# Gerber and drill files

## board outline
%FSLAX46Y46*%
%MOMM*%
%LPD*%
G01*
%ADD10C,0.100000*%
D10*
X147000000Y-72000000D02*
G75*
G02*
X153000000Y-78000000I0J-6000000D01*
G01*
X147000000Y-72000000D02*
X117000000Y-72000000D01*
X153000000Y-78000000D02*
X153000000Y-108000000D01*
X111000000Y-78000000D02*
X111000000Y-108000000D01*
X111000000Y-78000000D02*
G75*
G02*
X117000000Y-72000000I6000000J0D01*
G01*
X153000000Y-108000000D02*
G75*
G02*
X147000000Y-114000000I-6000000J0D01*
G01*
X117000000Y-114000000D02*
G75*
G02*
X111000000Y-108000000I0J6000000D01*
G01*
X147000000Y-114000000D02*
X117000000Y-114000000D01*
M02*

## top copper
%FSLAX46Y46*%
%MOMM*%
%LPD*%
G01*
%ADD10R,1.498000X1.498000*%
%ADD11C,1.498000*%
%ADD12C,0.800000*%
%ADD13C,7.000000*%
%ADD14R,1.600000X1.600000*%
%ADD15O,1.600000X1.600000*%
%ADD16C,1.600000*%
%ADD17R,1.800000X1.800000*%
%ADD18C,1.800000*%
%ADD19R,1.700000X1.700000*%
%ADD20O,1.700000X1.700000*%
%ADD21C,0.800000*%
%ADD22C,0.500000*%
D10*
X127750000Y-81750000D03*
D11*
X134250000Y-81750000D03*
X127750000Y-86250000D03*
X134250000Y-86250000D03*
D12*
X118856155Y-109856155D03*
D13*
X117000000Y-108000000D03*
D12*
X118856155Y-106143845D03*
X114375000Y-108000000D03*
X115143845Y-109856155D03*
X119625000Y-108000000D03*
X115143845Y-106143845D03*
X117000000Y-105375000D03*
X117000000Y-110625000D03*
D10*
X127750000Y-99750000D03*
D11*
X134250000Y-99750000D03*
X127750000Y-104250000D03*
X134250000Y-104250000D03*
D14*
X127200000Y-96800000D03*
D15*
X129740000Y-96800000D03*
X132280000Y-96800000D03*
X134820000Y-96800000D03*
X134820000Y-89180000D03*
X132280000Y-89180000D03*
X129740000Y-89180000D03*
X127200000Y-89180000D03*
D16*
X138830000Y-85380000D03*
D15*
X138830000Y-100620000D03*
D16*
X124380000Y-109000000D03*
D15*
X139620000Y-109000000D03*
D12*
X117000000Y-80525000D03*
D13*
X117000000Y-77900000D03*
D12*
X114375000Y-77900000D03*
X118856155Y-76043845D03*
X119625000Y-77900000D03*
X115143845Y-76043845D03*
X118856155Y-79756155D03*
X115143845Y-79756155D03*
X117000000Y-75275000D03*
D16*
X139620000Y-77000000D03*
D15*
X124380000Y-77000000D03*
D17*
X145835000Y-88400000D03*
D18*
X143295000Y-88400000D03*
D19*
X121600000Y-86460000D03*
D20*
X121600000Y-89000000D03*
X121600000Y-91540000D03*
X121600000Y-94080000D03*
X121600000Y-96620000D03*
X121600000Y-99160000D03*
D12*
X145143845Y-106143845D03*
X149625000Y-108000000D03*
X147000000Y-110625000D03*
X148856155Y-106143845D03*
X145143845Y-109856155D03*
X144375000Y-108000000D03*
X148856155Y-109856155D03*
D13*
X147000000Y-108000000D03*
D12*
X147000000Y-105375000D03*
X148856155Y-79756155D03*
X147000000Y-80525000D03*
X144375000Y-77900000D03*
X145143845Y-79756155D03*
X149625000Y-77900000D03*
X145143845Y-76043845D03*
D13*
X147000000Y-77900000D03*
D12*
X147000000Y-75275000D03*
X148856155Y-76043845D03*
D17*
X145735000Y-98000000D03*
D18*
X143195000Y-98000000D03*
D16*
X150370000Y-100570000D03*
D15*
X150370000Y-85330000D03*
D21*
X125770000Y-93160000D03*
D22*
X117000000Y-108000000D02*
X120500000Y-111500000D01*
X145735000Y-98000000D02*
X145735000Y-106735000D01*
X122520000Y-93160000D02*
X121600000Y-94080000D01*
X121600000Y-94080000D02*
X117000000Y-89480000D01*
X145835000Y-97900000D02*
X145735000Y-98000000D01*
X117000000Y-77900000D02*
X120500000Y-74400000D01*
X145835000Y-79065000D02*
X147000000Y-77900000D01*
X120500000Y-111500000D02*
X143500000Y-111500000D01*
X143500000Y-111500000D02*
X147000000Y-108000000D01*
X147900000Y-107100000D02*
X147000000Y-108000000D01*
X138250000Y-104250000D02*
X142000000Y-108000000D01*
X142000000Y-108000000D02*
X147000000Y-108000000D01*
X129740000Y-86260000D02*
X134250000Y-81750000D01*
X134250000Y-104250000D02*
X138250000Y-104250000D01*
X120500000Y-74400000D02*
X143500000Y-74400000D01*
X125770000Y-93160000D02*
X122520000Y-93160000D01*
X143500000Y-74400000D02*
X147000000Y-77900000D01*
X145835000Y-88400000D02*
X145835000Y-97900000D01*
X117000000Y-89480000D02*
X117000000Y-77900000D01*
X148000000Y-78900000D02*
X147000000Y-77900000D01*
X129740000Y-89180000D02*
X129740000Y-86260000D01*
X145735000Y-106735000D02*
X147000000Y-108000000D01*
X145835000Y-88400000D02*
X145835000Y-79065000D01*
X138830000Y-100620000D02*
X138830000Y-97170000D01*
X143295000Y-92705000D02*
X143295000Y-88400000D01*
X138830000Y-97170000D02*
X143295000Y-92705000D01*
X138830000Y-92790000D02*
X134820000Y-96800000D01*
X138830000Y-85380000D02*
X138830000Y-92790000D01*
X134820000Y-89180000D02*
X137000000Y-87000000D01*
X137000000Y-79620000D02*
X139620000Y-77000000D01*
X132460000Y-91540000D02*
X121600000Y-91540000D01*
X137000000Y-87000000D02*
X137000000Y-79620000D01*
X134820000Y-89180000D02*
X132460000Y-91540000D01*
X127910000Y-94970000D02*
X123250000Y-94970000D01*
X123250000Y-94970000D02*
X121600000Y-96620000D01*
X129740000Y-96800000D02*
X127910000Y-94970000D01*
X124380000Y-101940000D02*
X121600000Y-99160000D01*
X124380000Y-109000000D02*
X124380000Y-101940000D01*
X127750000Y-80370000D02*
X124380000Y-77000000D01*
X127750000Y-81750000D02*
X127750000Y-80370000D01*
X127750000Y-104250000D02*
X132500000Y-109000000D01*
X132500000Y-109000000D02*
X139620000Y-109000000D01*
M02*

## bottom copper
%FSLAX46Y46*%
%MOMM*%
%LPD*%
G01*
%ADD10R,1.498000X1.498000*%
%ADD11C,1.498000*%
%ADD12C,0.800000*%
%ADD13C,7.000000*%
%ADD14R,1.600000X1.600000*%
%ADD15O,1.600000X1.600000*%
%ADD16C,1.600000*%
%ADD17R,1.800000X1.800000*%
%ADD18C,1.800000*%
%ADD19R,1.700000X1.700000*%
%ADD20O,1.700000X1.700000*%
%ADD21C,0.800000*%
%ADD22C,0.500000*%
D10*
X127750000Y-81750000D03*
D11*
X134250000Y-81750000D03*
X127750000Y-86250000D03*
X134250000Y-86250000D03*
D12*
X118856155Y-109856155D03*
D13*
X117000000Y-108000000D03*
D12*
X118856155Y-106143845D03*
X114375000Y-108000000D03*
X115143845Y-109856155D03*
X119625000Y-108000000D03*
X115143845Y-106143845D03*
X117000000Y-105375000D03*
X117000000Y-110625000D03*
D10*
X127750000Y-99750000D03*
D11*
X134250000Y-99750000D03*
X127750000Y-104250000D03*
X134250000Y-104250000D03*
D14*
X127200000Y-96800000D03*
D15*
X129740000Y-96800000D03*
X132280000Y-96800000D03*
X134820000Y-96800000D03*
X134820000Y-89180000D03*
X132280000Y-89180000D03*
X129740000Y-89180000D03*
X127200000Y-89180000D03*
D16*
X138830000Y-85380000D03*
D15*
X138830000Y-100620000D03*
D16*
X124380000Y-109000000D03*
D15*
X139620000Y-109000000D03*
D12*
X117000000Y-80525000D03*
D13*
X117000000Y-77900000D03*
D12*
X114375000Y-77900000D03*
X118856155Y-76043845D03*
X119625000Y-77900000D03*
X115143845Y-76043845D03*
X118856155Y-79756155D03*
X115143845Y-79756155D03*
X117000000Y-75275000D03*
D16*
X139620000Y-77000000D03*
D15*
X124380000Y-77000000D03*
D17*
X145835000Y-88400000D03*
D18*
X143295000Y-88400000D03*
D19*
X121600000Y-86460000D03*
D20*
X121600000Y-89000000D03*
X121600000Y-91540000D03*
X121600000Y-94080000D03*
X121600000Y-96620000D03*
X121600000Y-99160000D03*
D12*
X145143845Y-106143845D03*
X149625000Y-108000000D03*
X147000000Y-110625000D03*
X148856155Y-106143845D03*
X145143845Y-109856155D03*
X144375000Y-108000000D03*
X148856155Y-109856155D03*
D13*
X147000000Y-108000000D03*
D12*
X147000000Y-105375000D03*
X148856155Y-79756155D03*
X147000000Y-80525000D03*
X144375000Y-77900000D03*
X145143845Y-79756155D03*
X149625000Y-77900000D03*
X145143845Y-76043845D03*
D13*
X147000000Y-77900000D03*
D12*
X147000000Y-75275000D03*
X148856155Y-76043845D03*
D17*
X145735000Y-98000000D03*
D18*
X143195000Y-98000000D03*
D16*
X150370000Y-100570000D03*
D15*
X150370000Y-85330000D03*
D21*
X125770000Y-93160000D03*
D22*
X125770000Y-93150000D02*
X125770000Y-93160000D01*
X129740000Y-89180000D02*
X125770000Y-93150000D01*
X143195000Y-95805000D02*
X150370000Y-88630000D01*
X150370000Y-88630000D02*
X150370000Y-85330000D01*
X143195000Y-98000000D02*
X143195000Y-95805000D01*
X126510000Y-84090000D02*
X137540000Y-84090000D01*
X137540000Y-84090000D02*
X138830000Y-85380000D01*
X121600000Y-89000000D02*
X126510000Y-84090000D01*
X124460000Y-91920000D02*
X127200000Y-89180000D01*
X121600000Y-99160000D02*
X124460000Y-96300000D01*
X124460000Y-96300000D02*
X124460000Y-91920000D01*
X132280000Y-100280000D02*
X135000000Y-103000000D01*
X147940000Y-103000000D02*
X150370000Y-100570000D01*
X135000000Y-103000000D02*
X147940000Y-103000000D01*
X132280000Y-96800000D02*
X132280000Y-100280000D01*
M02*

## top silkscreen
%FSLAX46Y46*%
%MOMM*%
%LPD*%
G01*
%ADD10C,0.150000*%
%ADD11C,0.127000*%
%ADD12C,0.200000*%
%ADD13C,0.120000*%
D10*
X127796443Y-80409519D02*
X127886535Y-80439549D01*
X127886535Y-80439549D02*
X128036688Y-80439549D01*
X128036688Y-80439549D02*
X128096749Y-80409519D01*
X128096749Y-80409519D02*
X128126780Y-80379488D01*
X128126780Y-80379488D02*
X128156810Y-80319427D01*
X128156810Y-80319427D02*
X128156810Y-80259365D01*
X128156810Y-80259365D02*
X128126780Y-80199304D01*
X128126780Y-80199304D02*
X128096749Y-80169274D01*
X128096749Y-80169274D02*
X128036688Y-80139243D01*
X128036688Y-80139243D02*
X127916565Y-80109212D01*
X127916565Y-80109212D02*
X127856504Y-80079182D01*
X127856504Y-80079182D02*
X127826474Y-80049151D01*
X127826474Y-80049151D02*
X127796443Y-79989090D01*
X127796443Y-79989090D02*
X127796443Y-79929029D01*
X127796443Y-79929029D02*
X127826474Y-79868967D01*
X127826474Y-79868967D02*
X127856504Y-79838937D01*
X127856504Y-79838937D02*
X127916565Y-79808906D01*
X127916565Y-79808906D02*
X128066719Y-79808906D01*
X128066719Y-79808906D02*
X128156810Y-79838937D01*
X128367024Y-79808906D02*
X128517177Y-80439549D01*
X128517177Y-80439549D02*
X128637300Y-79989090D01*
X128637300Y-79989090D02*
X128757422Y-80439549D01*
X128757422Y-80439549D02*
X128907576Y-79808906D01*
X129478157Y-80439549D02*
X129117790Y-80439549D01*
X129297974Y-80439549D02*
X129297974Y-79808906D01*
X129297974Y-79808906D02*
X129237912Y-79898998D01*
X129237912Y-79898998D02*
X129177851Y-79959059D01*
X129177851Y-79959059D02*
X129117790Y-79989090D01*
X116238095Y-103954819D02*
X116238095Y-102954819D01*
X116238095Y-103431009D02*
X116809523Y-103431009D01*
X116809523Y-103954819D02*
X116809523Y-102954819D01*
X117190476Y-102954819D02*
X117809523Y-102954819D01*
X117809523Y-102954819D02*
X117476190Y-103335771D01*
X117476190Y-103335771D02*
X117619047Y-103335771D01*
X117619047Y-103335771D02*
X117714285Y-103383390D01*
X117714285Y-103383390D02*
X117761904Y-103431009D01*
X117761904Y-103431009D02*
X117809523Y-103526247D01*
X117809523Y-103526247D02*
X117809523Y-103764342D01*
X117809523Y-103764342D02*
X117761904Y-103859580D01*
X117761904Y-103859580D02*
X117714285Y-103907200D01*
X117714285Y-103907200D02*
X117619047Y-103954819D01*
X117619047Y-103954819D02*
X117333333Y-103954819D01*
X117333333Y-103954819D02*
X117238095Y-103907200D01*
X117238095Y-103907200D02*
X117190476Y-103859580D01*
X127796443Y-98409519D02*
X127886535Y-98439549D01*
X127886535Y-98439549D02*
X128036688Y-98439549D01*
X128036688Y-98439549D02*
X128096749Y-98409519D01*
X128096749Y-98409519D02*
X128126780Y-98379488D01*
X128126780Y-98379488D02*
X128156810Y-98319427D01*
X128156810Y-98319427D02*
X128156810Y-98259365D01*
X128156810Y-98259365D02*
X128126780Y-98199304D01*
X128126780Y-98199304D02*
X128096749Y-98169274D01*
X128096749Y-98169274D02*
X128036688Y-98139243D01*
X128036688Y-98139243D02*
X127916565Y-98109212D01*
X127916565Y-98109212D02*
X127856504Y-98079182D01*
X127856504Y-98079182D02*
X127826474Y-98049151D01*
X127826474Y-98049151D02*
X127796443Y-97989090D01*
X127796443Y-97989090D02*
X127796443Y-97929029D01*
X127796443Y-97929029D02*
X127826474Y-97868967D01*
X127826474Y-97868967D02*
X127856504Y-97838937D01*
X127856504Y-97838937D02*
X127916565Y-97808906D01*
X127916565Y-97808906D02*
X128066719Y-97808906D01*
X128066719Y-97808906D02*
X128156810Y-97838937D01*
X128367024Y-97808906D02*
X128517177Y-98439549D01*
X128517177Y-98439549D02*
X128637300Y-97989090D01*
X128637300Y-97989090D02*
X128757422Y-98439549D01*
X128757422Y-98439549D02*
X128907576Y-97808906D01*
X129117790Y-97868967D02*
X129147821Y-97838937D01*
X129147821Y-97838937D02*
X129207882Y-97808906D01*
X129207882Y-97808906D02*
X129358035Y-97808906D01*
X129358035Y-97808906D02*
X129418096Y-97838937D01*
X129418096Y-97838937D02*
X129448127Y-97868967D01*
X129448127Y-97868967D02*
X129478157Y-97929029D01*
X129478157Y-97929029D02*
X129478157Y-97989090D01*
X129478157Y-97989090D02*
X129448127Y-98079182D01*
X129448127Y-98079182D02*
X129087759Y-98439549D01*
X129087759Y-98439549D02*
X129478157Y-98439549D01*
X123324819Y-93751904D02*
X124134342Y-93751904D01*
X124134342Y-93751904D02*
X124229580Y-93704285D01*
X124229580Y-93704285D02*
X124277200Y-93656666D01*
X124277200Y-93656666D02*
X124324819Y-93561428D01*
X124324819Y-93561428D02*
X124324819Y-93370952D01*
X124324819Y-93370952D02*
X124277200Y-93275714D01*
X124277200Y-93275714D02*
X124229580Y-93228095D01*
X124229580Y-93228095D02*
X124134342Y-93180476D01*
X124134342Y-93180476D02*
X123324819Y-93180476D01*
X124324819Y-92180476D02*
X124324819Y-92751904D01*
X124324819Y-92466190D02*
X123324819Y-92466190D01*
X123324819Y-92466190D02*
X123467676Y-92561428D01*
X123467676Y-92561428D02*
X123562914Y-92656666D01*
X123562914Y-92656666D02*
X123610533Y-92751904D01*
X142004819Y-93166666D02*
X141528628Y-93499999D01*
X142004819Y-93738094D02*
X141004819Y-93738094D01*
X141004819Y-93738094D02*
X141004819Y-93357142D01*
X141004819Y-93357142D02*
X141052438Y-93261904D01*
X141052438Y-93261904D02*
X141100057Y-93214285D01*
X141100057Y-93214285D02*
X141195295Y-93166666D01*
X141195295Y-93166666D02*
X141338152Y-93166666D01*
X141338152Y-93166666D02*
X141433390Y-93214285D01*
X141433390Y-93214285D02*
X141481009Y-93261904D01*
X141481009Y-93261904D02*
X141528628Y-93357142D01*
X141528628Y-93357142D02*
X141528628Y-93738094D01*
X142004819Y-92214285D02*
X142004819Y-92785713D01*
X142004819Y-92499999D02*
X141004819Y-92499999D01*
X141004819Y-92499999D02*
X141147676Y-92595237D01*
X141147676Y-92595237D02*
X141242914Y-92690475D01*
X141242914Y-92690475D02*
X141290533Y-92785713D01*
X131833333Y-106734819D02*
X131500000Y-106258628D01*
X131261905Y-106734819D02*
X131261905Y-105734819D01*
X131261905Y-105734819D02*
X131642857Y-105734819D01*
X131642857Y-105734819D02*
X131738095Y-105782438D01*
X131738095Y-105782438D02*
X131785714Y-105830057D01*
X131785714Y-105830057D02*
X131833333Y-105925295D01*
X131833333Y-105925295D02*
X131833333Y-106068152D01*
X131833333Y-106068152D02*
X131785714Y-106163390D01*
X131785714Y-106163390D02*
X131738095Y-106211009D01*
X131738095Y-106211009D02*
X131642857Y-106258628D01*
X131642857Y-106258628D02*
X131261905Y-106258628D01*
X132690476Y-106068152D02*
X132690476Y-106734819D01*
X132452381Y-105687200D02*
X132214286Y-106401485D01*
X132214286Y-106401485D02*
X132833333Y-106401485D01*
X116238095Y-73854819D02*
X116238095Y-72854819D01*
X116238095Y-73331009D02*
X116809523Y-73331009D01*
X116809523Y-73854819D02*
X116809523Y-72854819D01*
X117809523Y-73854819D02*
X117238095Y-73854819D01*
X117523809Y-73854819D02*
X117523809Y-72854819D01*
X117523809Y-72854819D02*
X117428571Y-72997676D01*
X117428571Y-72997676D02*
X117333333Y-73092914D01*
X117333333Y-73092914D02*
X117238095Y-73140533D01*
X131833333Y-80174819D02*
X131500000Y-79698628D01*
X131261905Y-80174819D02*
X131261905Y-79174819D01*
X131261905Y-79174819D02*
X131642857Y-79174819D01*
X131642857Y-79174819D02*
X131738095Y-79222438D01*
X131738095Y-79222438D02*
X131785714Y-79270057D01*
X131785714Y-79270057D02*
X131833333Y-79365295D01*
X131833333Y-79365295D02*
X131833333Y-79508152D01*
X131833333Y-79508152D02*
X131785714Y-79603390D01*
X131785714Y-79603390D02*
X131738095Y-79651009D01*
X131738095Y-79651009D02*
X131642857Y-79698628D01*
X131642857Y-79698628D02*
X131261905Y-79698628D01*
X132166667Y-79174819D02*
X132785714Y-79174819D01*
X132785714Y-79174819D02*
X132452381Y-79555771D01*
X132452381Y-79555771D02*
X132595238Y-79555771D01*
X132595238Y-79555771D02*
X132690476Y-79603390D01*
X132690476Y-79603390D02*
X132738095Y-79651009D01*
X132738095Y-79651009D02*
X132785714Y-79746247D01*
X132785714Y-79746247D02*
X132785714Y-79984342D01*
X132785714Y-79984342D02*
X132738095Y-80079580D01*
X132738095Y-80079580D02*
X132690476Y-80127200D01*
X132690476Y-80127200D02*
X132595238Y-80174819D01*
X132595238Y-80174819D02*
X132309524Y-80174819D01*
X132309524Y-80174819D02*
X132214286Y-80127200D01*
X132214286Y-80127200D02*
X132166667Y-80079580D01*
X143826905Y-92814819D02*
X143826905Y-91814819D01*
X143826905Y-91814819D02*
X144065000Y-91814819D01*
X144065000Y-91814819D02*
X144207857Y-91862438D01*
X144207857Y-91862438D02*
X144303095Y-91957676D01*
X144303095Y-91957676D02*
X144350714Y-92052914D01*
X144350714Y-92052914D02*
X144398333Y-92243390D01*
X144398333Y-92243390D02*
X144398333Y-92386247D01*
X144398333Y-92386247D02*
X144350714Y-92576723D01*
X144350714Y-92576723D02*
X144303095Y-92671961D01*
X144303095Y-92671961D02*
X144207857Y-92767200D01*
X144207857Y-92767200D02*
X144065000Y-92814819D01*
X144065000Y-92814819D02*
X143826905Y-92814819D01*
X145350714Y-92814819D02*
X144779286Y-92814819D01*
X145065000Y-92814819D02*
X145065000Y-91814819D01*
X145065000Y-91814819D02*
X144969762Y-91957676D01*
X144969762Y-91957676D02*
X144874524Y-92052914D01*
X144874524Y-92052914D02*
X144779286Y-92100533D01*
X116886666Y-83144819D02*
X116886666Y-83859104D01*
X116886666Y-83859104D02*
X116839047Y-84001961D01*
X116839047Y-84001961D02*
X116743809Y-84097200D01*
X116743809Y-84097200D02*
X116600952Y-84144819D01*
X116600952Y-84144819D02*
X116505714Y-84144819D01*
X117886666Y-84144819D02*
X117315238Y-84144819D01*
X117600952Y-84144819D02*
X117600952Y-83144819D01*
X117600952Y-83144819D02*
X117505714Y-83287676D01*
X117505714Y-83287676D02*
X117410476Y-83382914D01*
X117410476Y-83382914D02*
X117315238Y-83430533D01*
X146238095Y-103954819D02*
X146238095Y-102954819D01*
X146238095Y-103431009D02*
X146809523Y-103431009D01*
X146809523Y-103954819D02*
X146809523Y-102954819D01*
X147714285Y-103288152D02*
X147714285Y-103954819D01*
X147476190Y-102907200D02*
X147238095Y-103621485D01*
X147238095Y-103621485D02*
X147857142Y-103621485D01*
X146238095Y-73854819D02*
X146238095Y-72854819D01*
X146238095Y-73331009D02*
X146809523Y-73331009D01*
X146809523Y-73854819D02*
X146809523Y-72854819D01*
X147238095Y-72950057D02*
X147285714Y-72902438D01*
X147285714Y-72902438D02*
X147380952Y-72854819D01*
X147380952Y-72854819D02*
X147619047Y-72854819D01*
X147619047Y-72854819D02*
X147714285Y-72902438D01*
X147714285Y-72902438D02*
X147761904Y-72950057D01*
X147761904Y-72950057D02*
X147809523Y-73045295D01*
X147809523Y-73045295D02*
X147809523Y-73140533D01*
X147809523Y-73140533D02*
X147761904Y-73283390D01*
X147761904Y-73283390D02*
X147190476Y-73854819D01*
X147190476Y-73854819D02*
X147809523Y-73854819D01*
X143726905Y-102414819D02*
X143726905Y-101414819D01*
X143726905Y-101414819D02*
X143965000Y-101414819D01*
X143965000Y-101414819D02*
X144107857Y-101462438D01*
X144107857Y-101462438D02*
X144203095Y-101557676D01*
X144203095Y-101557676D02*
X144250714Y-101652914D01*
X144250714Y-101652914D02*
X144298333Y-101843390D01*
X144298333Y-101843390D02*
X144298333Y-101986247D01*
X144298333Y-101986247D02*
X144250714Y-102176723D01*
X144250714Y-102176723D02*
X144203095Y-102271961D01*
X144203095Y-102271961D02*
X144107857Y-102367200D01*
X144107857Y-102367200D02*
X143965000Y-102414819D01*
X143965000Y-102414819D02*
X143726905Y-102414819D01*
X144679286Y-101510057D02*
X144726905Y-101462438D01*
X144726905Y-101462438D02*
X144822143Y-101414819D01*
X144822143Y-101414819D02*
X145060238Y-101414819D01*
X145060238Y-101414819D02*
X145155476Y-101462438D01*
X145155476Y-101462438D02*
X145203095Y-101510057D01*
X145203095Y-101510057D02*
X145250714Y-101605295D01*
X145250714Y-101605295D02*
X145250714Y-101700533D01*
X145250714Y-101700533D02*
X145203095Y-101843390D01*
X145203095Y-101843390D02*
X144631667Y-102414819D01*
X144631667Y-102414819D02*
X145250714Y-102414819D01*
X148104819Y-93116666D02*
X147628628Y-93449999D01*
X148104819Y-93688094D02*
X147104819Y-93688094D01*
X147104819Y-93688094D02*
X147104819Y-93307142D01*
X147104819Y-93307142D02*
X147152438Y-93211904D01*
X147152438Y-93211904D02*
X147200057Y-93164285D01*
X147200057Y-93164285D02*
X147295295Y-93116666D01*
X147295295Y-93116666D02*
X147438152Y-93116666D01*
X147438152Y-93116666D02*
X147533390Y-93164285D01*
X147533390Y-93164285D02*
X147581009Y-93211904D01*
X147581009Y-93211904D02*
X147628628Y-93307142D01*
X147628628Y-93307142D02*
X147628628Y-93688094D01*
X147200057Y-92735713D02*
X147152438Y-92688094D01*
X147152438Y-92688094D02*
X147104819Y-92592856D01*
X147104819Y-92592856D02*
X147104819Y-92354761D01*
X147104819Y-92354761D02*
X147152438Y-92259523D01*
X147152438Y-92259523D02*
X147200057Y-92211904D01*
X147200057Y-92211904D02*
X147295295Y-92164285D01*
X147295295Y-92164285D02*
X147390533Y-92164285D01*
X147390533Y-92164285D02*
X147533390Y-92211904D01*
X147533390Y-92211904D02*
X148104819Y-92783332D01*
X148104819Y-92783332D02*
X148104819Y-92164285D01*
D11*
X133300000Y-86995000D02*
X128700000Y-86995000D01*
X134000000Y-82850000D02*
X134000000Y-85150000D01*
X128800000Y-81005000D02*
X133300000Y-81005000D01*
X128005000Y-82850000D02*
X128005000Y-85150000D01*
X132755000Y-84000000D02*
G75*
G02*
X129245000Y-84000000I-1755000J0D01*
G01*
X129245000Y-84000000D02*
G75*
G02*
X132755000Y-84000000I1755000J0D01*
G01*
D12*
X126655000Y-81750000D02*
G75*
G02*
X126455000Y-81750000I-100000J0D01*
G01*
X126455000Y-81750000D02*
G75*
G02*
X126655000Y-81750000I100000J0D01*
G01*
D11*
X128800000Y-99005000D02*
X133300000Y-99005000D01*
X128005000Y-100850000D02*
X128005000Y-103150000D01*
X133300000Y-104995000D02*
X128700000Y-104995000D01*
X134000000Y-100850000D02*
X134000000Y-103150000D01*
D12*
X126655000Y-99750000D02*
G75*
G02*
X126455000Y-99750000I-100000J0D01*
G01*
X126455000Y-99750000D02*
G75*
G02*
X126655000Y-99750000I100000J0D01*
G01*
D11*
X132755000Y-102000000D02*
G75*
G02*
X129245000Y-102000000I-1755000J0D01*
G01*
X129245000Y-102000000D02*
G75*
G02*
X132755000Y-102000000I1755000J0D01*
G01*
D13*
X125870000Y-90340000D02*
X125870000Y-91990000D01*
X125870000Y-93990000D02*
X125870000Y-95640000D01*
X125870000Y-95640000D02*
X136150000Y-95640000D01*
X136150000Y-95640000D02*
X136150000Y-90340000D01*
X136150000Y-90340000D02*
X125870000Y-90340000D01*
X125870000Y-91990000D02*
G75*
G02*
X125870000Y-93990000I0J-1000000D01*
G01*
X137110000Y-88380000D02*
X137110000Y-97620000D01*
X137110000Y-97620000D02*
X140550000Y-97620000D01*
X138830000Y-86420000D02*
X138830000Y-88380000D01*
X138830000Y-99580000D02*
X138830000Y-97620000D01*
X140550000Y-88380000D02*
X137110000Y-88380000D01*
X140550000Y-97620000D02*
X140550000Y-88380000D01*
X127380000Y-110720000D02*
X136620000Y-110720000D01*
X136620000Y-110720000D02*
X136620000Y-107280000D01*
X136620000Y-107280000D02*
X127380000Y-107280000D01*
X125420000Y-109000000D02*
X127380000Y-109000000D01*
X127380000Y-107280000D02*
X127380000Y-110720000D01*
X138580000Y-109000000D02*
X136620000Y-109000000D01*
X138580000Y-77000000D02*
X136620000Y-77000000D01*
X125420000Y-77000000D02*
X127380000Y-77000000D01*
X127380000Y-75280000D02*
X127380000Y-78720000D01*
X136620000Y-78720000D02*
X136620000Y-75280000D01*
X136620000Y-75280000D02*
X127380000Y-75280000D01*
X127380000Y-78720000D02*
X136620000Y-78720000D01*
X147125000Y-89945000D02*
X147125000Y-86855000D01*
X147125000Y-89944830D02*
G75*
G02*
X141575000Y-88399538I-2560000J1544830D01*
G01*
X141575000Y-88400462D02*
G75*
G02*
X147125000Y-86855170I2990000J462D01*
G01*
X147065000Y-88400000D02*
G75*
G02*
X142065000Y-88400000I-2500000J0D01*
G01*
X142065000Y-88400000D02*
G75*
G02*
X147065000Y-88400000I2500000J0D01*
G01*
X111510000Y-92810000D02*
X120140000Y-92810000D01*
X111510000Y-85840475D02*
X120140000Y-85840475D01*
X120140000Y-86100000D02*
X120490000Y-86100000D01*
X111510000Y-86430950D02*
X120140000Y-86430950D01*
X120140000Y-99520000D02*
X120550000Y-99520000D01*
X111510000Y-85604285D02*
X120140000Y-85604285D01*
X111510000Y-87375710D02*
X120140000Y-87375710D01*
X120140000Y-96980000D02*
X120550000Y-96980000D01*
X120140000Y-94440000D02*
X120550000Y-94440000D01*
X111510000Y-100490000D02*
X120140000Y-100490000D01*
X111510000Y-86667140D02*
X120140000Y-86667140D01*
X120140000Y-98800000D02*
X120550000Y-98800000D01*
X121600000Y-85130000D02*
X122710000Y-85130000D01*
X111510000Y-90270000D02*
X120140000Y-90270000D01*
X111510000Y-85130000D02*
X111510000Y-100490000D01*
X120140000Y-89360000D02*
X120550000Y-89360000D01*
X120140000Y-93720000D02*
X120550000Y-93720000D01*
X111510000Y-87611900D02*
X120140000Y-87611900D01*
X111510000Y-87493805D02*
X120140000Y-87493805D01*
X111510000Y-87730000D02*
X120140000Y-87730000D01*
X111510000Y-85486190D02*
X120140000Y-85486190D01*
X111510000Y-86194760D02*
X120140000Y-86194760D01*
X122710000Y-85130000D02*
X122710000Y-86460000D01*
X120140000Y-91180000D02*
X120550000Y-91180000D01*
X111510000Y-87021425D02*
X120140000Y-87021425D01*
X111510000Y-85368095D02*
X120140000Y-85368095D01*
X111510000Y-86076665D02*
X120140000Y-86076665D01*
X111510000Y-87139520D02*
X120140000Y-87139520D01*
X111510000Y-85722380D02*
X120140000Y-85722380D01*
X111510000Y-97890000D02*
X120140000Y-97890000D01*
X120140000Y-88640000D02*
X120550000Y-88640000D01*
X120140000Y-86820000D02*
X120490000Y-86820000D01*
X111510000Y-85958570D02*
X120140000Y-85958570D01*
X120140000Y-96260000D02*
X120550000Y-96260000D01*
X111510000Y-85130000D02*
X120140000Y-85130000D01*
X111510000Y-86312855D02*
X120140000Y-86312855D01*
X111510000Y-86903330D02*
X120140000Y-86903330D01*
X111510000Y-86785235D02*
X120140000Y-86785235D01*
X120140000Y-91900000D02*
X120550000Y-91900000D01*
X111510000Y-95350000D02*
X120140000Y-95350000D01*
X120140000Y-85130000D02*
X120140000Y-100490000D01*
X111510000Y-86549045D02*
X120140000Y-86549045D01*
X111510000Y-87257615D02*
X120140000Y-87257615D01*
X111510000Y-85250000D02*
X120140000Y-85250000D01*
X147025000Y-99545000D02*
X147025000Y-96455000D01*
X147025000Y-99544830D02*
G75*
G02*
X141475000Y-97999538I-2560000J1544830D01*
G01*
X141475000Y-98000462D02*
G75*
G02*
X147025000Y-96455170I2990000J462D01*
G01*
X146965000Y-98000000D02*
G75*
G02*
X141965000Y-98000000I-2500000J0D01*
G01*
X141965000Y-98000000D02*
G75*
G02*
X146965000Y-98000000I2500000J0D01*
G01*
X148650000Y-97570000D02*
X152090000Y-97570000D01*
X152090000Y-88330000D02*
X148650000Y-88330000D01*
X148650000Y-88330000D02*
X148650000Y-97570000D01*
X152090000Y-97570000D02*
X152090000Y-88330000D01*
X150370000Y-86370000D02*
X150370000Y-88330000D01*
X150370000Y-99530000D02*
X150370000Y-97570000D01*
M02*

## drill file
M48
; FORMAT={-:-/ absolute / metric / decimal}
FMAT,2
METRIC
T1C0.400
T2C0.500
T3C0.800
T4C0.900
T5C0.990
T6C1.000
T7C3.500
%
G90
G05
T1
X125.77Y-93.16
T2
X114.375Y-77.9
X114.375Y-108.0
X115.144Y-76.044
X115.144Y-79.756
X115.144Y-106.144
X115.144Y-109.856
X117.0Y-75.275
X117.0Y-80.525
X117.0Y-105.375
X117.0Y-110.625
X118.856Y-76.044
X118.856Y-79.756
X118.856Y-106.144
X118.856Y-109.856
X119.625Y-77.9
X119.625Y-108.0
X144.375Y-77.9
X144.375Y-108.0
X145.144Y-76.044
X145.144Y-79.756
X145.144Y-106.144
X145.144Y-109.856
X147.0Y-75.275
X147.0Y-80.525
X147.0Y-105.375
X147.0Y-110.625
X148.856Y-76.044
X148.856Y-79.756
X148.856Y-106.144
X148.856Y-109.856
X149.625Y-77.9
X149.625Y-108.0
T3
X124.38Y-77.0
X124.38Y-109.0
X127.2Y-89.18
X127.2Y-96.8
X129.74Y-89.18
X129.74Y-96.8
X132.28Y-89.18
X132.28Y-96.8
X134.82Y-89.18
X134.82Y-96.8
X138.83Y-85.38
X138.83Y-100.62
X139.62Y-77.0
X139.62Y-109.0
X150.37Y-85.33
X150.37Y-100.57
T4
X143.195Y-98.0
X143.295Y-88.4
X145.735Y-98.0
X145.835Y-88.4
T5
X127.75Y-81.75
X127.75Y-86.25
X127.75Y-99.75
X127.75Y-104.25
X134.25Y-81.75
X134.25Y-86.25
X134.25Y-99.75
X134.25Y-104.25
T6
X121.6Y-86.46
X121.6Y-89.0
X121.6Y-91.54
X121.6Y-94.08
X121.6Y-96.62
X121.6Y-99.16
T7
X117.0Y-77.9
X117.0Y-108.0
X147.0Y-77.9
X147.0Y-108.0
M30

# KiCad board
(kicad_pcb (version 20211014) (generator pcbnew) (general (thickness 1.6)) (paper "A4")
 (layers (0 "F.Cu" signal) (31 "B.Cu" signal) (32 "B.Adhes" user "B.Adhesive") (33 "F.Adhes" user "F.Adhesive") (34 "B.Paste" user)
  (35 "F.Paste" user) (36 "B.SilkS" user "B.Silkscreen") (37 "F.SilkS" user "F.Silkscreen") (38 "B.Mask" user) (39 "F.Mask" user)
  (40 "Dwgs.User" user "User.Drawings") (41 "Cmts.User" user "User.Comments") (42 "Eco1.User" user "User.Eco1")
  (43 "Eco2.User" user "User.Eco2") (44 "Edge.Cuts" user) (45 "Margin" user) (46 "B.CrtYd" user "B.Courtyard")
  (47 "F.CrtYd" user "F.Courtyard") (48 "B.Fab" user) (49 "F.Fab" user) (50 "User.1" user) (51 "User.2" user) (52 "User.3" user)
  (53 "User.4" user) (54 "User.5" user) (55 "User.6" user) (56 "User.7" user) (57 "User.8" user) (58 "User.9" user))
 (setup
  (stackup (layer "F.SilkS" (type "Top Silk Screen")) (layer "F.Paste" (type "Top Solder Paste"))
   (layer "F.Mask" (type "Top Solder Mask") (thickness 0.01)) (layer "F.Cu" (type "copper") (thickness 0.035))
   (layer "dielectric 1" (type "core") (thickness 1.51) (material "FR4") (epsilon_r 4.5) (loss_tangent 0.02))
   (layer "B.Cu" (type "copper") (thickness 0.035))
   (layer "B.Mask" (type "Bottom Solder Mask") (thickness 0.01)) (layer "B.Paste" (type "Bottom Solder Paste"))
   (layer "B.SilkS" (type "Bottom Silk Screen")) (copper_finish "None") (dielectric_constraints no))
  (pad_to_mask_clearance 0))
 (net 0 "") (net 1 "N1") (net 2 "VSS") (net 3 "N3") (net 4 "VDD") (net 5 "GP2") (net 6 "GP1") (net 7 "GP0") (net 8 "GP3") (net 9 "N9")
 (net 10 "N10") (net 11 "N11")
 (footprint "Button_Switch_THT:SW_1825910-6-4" (layer "F.Cu") (at 131 84)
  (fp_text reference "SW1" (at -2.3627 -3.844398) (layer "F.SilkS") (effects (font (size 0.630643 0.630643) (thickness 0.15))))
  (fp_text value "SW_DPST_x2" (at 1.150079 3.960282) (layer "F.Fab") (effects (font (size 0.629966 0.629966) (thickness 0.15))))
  (fp_line (start 2.3 2.995) (end -2.3 2.995) (layer "F.SilkS") (width 0.127))
  (fp_line (start 3 -1.15) (end 3 1.15) (layer "F.SilkS") (width 0.127))
  (fp_line (start -2.2 -2.995) (end 2.3 -2.995) (layer "F.SilkS") (width 0.127))
  (fp_line (start -2.995 -1.15) (end -2.995 1.15) (layer "F.SilkS") (width 0.127))
  (fp_circle (center 0 0) (end 1.755 0) (layer "F.SilkS") (width 0.127) (fill none))
  (fp_circle (center -4.445 -2.25) (end -4.345 -2.25) (layer "F.SilkS") (width 0.2) (fill none))
  (pad "1" thru_hole rect locked (at -3.25 -2.25) (size 1.498 1.498) (drill 0.99) (layers *.Cu *.Mask) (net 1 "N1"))
  (pad "2" thru_hole circle locked (at 3.25 -2.25) (size 1.498 1.498) (drill 0.99) (layers *.Cu *.Mask) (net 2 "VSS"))
  (pad "3" thru_hole circle locked (at -3.25 2.25) (size 1.498 1.498) (drill 0.99) (layers *.Cu *.Mask))
  (pad "4" thru_hole circle locked (at 3.25 2.25) (size 1.498 1.498) (drill 0.99) (layers *.Cu *.Mask)))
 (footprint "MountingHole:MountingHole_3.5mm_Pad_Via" (layer "F.Cu") (at 117 108)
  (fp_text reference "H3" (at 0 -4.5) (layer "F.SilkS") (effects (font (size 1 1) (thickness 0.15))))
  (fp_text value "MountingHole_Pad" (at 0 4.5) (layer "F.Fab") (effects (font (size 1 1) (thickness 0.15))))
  (pad "1" thru_hole circle (at 1.856155 1.856155) (size 0.8 0.8) (drill 0.5) (layers *.Cu *.Mask) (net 2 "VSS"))
  (pad "1" thru_hole circle (at 0 0) (size 7 7) (drill 3.5) (layers *.Cu *.Mask) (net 2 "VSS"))
  (pad "1" thru_hole circle (at 1.856155 -1.856155) (size 0.8 0.8) (drill 0.5) (layers *.Cu *.Mask) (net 2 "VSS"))
  (pad "1" thru_hole circle (at -2.625 0) (size 0.8 0.8) (drill 0.5) (layers *.Cu *.Mask) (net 2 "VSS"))
  (pad "1" thru_hole circle (at -1.856155 1.856155) (size 0.8 0.8) (drill 0.5) (layers *.Cu *.Mask) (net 2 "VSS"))
  (pad "1" thru_hole circle (at 2.625 0) (size 0.8 0.8) (drill 0.5) (layers *.Cu *.Mask) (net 2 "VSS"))
  (pad "1" thru_hole circle (at -1.856155 -1.856155) (size 0.8 0.8) (drill 0.5) (layers *.Cu *.Mask) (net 2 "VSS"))
  (pad "1" thru_hole circle (at 0 -2.625) (size 0.8 0.8) (drill 0.5) (layers *.Cu *.Mask) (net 2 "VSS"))
  (pad "1" thru_hole circle (at 0 2.625) (size 0.8 0.8) (drill 0.5) (layers *.Cu *.Mask) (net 2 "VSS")))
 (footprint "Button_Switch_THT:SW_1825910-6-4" (layer "F.Cu") (at 131 102)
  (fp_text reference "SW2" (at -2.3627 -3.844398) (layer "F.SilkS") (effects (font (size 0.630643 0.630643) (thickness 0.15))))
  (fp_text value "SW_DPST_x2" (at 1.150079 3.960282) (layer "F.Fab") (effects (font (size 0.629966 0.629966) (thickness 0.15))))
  (fp_line (start -2.2 -2.995) (end 2.3 -2.995) (layer "F.SilkS") (width 0.127))
  (fp_line (start -2.995 -1.15) (end -2.995 1.15) (layer "F.SilkS") (width 0.127))
  (fp_line (start 2.3 2.995) (end -2.3 2.995) (layer "F.SilkS") (width 0.127))
  (fp_line (start 3 -1.15) (end 3 1.15) (layer "F.SilkS") (width 0.127))
  (fp_circle (center -4.445 -2.25) (end -4.345 -2.25) (layer "F.SilkS") (width 0.2) (fill none))
  (fp_circle (center 0 0) (end 1.755 0) (layer "F.SilkS") (width 0.127) (fill none))
  (pad "1" thru_hole rect locked (at -3.25 -2.25) (size 1.498 1.498) (drill 0.99) (layers *.Cu *.Mask))
  (pad "2" thru_hole circle locked (at 3.25 -2.25) (size 1.498 1.498) (drill 0.99) (layers *.Cu *.Mask))
  (pad "3" thru_hole circle locked (at -3.25 2.25) (size 1.498 1.498) (drill 0.99) (layers *.Cu *.Mask) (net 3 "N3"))
  (pad "4" thru_hole circle locked (at 3.25 2.25) (size 1.498 1.498) (drill 0.99) (layers *.Cu *.Mask) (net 2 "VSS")))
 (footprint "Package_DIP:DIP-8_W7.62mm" (layer "F.Cu") (at 127.2 96.8 90)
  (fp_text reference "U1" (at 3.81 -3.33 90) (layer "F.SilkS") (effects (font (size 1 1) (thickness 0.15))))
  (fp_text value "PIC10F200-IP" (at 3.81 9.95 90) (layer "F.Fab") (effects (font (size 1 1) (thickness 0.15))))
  (fp_line (start 6.46 -1.33) (end 4.81 -1.33) (layer "F.SilkS") (width 0.12))
  (fp_line (start 2.81 -1.33) (end 1.16 -1.33) (layer "F.SilkS") (width 0.12))
  (fp_line (start 1.16 -1.33) (end 1.16 8.95) (layer "F.SilkS") (width 0.12))
  (fp_line (start 1.16 8.95) (end 6.46 8.95) (layer "F.SilkS") (width 0.12))
  (fp_line (start 6.46 8.95) (end 6.46 -1.33) (layer "F.SilkS") (width 0.12))
  (fp_arc (start 4.81 -1.33) (mid 3.81 -0.33) (end 2.81 -1.33) (layer "F.SilkS") (width 0.12))
  (pad "1" thru_hole rect (at 0 0 90) (size 1.6 1.6) (drill 0.8) (layers *.Cu *.Mask))
  (pad "2" thru_hole oval (at 0 2.54 90) (size 1.6 1.6) (drill 0.8) (layers *.Cu *.Mask) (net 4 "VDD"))
  (pad "3" thru_hole oval (at 0 5.08 90) (size 1.6 1.6) (drill 0.8) (layers *.Cu *.Mask) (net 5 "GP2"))
  (pad "4" thru_hole oval (at 0 7.62 90) (size 1.6 1.6) (drill 0.8) (layers *.Cu *.Mask) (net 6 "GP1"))
  (pad "5" thru_hole oval (at 7.62 7.62 90) (size 1.6 1.6) (drill 0.8) (layers *.Cu *.Mask) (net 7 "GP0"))
  (pad "6" thru_hole oval (at 7.62 5.08 90) (size 1.6 1.6) (drill 0.8) (layers *.Cu *.Mask))
  (pad "7" thru_hole oval (at 7.62 2.54 90) (size 1.6 1.6) (drill 0.8) (layers *.Cu *.Mask) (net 2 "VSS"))
  (pad "8" thru_hole oval (at 7.62 0 90) (size 1.6 1.6) (drill 0.8) (layers *.Cu *.Mask) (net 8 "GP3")))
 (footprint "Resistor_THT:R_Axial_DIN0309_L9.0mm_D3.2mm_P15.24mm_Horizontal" (layer "F.Cu") (at 138.83 85.38 -90)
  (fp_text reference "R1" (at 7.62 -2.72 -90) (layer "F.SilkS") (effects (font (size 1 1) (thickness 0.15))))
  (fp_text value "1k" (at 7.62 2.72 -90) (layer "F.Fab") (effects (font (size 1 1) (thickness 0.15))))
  (fp_line (start 3 1.72) (end 12.24 1.72) (layer "F.SilkS") (width 0.12))
  (fp_line (start 12.24 1.72) (end 12.24 -1.72) (layer "F.SilkS") (width 0.12))
  (fp_line (start 1.04 0) (end 3 0) (layer "F.SilkS") (width 0.12))
  (fp_line (start 14.2 0) (end 12.24 0) (layer "F.SilkS") (width 0.12))
  (fp_line (start 3 -1.72) (end 3 1.72) (layer "F.SilkS") (width 0.12))
  (fp_line (start 12.24 -1.72) (end 3 -1.72) (layer "F.SilkS") (width 0.12))
  (pad "1" thru_hole circle (at 0 0 270) (size 1.6 1.6) (drill 0.8) (layers *.Cu *.Mask) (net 6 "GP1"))
  (pad "2" thru_hole oval (at 15.24 0 270) (size 1.6 1.6) (drill 0.8) (layers *.Cu *.Mask) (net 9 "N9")))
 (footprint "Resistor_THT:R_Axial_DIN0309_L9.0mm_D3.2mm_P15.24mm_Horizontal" (layer "F.Cu") (at 124.38 109)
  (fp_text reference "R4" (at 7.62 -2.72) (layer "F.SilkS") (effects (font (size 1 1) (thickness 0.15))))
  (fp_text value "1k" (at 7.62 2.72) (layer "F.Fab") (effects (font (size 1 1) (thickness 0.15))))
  (fp_line (start 3 1.72) (end 12.24 1.72) (layer "F.SilkS") (width 0.12))
  (fp_line (start 12.24 1.72) (end 12.24 -1.72) (layer "F.SilkS") (width 0.12))
  (fp_line (start 12.24 -1.72) (end 3 -1.72) (layer "F.SilkS") (width 0.12))
  (fp_line (start 1.04 0) (end 3 0) (layer "F.SilkS") (width 0.12))
  (fp_line (start 3 -1.72) (end 3 1.72) (layer "F.SilkS") (width 0.12))
  (fp_line (start 14.2 0) (end 12.24 0) (layer "F.SilkS") (width 0.12))
  (pad "1" thru_hole circle (at 0 0) (size 1.6 1.6) (drill 0.8) (layers *.Cu *.Mask) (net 8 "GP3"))
  (pad "2" thru_hole oval (at 15.24 0) (size 1.6 1.6) (drill 0.8) (layers *.Cu *.Mask) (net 3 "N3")))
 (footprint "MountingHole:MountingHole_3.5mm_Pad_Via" (layer "F.Cu") (at 117 77.9)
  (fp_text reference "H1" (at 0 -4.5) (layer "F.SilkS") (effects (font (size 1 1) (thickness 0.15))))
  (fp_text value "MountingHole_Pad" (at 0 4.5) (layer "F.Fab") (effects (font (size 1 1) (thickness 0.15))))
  (pad "1" thru_hole circle (at 0 2.625) (size 0.8 0.8) (drill 0.5) (layers *.Cu *.Mask) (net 2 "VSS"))
  (pad "1" thru_hole circle (at 0 0) (size 7 7) (drill 3.5) (layers *.Cu *.Mask) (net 2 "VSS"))
  (pad "1" thru_hole circle (at -2.625 0) (size 0.8 0.8) (drill 0.5) (layers *.Cu *.Mask) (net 2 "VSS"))
  (pad "1" thru_hole circle (at 1.856155 -1.856155) (size 0.8 0.8) (drill 0.5) (layers *.Cu *.Mask) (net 2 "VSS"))
  (pad "1" thru_hole circle (at 2.625 0) (size 0.8 0.8) (drill 0.5) (layers *.Cu *.Mask) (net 2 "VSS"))
  (pad "1" thru_hole circle (at -1.856155 -1.856155) (size 0.8 0.8) (drill 0.5) (layers *.Cu *.Mask) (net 2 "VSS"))
  (pad "1" thru_hole circle (at 1.856155 1.856155) (size 0.8 0.8) (drill 0.5) (layers *.Cu *.Mask) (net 2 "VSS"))
  (pad "1" thru_hole circle (at -1.856155 1.856155) (size 0.8 0.8) (drill 0.5) (layers *.Cu *.Mask) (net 2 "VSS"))
  (pad "1" thru_hole circle (at 0 -2.625) (size 0.8 0.8) (drill 0.5) (layers *.Cu *.Mask) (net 2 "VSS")))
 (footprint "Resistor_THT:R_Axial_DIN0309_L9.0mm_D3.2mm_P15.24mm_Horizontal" (layer "F.Cu") (at 139.62 77 180)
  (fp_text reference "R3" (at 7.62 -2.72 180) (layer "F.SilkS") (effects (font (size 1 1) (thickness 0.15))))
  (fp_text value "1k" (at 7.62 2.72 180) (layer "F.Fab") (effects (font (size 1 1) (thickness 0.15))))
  (fp_line (start 1.04 0) (end 3 0) (layer "F.SilkS") (width 0.12))
  (fp_line (start 14.2 0) (end 12.24 0) (layer "F.SilkS") (width 0.12))
  (fp_line (start 12.24 1.72) (end 12.24 -1.72) (layer "F.SilkS") (width 0.12))
  (fp_line (start 3 -1.72) (end 3 1.72) (layer "F.SilkS") (width 0.12))
  (fp_line (start 3 1.72) (end 12.24 1.72) (layer "F.SilkS") (width 0.12))
  (fp_line (start 12.24 -1.72) (end 3 -1.72) (layer "F.SilkS") (width 0.12))
  (pad "1" thru_hole circle (at 0 0 180) (size 1.6 1.6) (drill 0.8) (layers *.Cu *.Mask) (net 7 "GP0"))
  (pad "2" thru_hole oval (at 15.24 0 180) (size 1.6 1.6) (drill 0.8) (layers *.Cu *.Mask) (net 1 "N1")))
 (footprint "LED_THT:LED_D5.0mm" (layer "F.Cu") (at 145.835 88.4 180)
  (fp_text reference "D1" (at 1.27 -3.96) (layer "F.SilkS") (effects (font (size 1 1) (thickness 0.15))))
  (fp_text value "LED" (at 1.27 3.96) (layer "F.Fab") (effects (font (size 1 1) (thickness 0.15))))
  (fp_line (start -1.29 -1.545) (end -1.29 1.545) (layer "F.SilkS") (width 0.12))
  (fp_arc (start -1.29 -1.54483) (mid 2.072002 -2.880433) (end 4.26 0.000462) (layer "F.SilkS") (width 0.12))
  (fp_arc (start 4.26 -0.000462) (mid 2.072002 2.880433) (end -1.29 1.54483) (layer "F.SilkS") (width 0.12))
  (fp_circle (center 1.27 0) (end 3.77 0) (layer "F.SilkS") (width 0.12) (fill none))
  (pad "1" thru_hole rect (at 0 0 180) (size 1.8 1.8) (drill 0.9) (layers *.Cu *.Mask) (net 2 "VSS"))
  (pad "2" thru_hole circle (at 2.54 0 180) (size 1.8 1.8) (drill 0.9) (layers *.Cu *.Mask) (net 9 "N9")))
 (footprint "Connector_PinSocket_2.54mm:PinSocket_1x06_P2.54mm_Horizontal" (layer "F.Cu") (at 121.6 86.46)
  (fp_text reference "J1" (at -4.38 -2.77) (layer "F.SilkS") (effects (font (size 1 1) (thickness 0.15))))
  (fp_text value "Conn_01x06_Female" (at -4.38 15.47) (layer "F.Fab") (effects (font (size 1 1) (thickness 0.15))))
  (fp_line (start -10.09 6.35) (end -1.46 6.35) (layer "F.SilkS") (width 0.12))
  (fp_line (start -10.09 -0.619525) (end -1.46 -0.619525) (layer "F.SilkS") (width 0.12))
  (fp_line (start -1.46 -0.36) (end -1.11 -0.36) (layer "F.SilkS") (width 0.12))
  (fp_line (start -10.09 -0.02905) (end -1.46 -0.02905) (layer "F.SilkS") (width 0.12))
  (fp_line (start -1.46 13.06) (end -1.05 13.06) (layer "F.SilkS") (width 0.12))
  (fp_line (start -10.09 -0.855715) (end -1.46 -0.855715) (layer "F.SilkS") (width 0.12))
  (fp_line (start -10.09 0.91571) (end -1.46 0.91571) (layer "F.SilkS") (width 0.12))
  (fp_line (start -1.46 10.52) (end -1.05 10.52) (layer "F.SilkS") (width 0.12))
  (fp_line (start -1.46 7.98) (end -1.05 7.98) (layer "F.SilkS") (width 0.12))
  (fp_line (start -10.09 14.03) (end -1.46 14.03) (layer "F.SilkS") (width 0.12))
  (fp_line (start -10.09 0.20714) (end -1.46 0.20714) (layer "F.SilkS") (width 0.12))
  (fp_line (start -1.46 12.34) (end -1.05 12.34) (layer "F.SilkS") (width 0.12))
  (fp_line (start 0 -1.33) (end 1.11 -1.33) (layer "F.SilkS") (width 0.12))
  (fp_line (start -10.09 3.81) (end -1.46 3.81) (layer "F.SilkS") (width 0.12))
  (fp_line (start -10.09 -1.33) (end -10.09 14.03) (layer "F.SilkS") (width 0.12))
  (fp_line (start -1.46 2.9) (end -1.05 2.9) (layer "F.SilkS") (width 0.12))
  (fp_line (start -1.46 7.26) (end -1.05 7.26) (layer "F.SilkS") (width 0.12))
  (fp_line (start -10.09 1.1519) (end -1.46 1.1519) (layer "F.SilkS") (width 0.12))
  (fp_line (start -10.09 1.033805) (end -1.46 1.033805) (layer "F.SilkS") (width 0.12))
  (fp_line (start -10.09 1.27) (end -1.46 1.27) (layer "F.SilkS") (width 0.12))
  (fp_line (start -10.09 -0.97381) (end -1.46 -0.97381) (layer "F.SilkS") (width 0.12))
  (fp_line (start -10.09 -0.26524) (end -1.46 -0.26524) (layer "F.SilkS") (width 0.12))
  (fp_line (start 1.11 -1.33) (end 1.11 0) (layer "F.SilkS") (width 0.12))
  (fp_line (start -1.46 4.72) (end -1.05 4.72) (layer "F.SilkS") (width 0.12))
  (fp_line (start -10.09 0.561425) (end -1.46 0.561425) (layer "F.SilkS") (width 0.12))
  (fp_line (start -10.09 -1.091905) (end -1.46 -1.091905) (layer "F.SilkS") (width 0.12))
  (fp_line (start -10.09 -0.383335) (end -1.46 -0.383335) (layer "F.SilkS") (width 0.12))
  (fp_line (start -10.09 0.67952) (end -1.46 0.67952) (layer "F.SilkS") (width 0.12))
  (fp_line (start -10.09 -0.73762) (end -1.46 -0.73762) (layer "F.SilkS") (width 0.12))
  (fp_line (start -10.09 11.43) (end -1.46 11.43) (layer "F.SilkS") (width 0.12))
  (fp_line (start -1.46 2.18) (end -1.05 2.18) (layer "F.SilkS") (width 0.12))
  (fp_line (start -1.46 0.36) (end -1.11 0.36) (layer "F.SilkS") (width 0.12))
  (fp_line (start -10.09 -0.50143) (end -1.46 -0.50143) (layer "F.SilkS") (width 0.12))
  (fp_line (start -1.46 9.8) (end -1.05 9.8) (layer "F.SilkS") (width 0.12))
  (fp_line (start -10.09 -1.33) (end -1.46 -1.33) (layer "F.SilkS") (width 0.12))
  (fp_line (start -10.09 -0.147145) (end -1.46 -0.147145) (layer "F.SilkS") (width 0.12))
  (fp_line (start -10.09 0.44333) (end -1.46 0.44333) (layer "F.SilkS") (width 0.12))
  (fp_line (start -10.09 0.325235) (end -1.46 0.325235) (layer "F.SilkS") (width 0.12))
  (fp_line (start -1.46 5.44) (end -1.05 5.44) (layer "F.SilkS") (width 0.12))
  (fp_line (start -10.09 8.89) (end -1.46 8.89) (layer "F.SilkS") (width 0.12))
  (fp_line (start -1.46 -1.33) (end -1.46 14.03) (layer "F.SilkS") (width 0.12))
  (fp_line (start -10.09 0.089045) (end -1.46 0.089045) (layer "F.SilkS") (width 0.12))
  (fp_line (start -10.09 0.797615) (end -1.46 0.797615) (layer "F.SilkS") (width 0.12))
  (fp_line (start -10.09 -1.21) (end -1.46 -1.21) (layer "F.SilkS") (width 0.12))
  (pad "1" thru_hole rect (at 0 0) (size 1.7 1.7) (drill 1) (layers *.Cu *.Mask) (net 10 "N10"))
  (pad "2" thru_hole oval (at 0 2.54) (size 1.7 1.7) (drill 1) (layers *.Cu *.Mask) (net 6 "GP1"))
  (pad "3" thru_hole oval (at 0 5.08) (size 1.7 1.7) (drill 1) (layers *.Cu *.Mask) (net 7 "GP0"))
  (pad "4" thru_hole oval (at 0 7.62) (size 1.7 1.7) (drill 1) (layers *.Cu *.Mask) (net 2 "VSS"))
  (pad "5" thru_hole oval (at 0 10.16) (size 1.7 1.7) (drill 1) (layers *.Cu *.Mask) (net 4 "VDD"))
  (pad "6" thru_hole oval (at 0 12.7) (size 1.7 1.7) (drill 1) (layers *.Cu *.Mask) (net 8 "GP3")))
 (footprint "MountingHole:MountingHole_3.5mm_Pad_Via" (layer "F.Cu") (at 147 108)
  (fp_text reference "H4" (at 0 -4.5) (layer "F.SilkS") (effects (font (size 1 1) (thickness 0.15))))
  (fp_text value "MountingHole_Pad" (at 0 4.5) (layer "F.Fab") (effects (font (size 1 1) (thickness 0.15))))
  (pad "1" thru_hole circle (at -1.856155 -1.856155) (size 0.8 0.8) (drill 0.5) (layers *.Cu *.Mask) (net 2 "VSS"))
  (pad "1" thru_hole circle (at 2.625 0) (size 0.8 0.8) (drill 0.5) (layers *.Cu *.Mask) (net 2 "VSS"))
  (pad "1" thru_hole circle (at 0 2.625) (size 0.8 0.8) (drill 0.5) (layers *.Cu *.Mask) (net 2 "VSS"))
  (pad "1" thru_hole circle (at 1.856155 -1.856155) (size 0.8 0.8) (drill 0.5) (layers *.Cu *.Mask) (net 2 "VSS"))
  (pad "1" thru_hole circle (at -1.856155 1.856155) (size 0.8 0.8) (drill 0.5) (layers *.Cu *.Mask) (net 2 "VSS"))
  (pad "1" thru_hole circle (at -2.625 0) (size 0.8 0.8) (drill 0.5) (layers *.Cu *.Mask) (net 2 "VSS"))
  (pad "1" thru_hole circle (at 1.856155 1.856155) (size 0.8 0.8) (drill 0.5) (layers *.Cu *.Mask) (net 2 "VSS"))
  (pad "1" thru_hole circle (at 0 0) (size 7 7) (drill 3.5) (layers *.Cu *.Mask) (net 2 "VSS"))
  (pad "1" thru_hole circle (at 0 -2.625) (size 0.8 0.8) (drill 0.5) (layers *.Cu *.Mask) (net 2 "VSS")))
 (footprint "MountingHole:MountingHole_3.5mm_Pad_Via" (layer "F.Cu") (at 147 77.9)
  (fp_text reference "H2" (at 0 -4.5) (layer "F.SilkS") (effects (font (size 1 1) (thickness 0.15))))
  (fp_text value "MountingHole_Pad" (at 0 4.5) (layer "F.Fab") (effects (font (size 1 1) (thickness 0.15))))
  (pad "1" thru_hole circle (at 1.856155 1.856155) (size 0.8 0.8) (drill 0.5) (layers *.Cu *.Mask) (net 2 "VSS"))
  (pad "1" thru_hole circle (at 0 2.625) (size 0.8 0.8) (drill 0.5) (layers *.Cu *.Mask) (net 2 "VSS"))
  (pad "1" thru_hole circle (at -2.625 0) (size 0.8 0.8) (drill 0.5) (layers *.Cu *.Mask) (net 2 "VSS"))
  (pad "1" thru_hole circle (at -1.856155 1.856155) (size 0.8 0.8) (drill 0.5) (layers *.Cu *.Mask) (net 2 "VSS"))
  (pad "1" thru_hole circle (at 2.625 0) (size 0.8 0.8) (drill 0.5) (layers *.Cu *.Mask) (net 2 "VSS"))
  (pad "1" thru_hole circle (at -1.856155 -1.856155) (size 0.8 0.8) (drill 0.5) (layers *.Cu *.Mask) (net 2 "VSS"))
  (pad "1" thru_hole circle (at 0 0) (size 7 7) (drill 3.5) (layers *.Cu *.Mask) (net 2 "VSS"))
  (pad "1" thru_hole circle (at 0 -2.625) (size 0.8 0.8) (drill 0.5) (layers *.Cu *.Mask) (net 2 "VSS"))
  (pad "1" thru_hole circle (at 1.856155 -1.856155) (size 0.8 0.8) (drill 0.5) (layers *.Cu *.Mask) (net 2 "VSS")))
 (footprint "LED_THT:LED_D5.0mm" (layer "F.Cu") (at 145.735 98 180)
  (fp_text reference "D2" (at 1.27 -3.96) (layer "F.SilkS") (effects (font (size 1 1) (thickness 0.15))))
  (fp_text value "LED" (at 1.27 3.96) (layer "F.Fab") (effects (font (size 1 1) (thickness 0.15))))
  (fp_line (start -1.29 -1.545) (end -1.29 1.545) (layer "F.SilkS") (width 0.12))
  (fp_arc (start -1.29 -1.54483) (mid 2.072002 -2.880433) (end 4.26 0.000462) (layer "F.SilkS") (width 0.12))
  (fp_arc (start 4.26 -0.000462) (mid 2.072002 2.880433) (end -1.29 1.54483) (layer "F.SilkS") (width 0.12))
  (fp_circle (center 1.27 0) (end 3.77 0) (layer "F.SilkS") (width 0.12) (fill none))
  (pad "1" thru_hole rect (at 0 0 180) (size 1.8 1.8) (drill 0.9) (layers *.Cu *.Mask) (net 2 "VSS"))
  (pad "2" thru_hole circle (at 2.54 0 180) (size 1.8 1.8) (drill 0.9) (layers *.Cu *.Mask) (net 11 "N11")))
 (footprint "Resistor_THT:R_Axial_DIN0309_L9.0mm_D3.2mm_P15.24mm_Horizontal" (layer "F.Cu") (at 150.37 100.57 90)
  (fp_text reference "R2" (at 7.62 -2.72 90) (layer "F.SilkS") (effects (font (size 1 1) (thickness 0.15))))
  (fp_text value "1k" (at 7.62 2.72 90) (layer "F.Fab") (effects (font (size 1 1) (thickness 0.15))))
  (fp_line (start 3 -1.72) (end 3 1.72) (layer "F.SilkS") (width 0.12))
  (fp_line (start 12.24 1.72) (end 12.24 -1.72) (layer "F.SilkS") (width 0.12))
  (fp_line (start 12.24 -1.72) (end 3 -1.72) (layer "F.SilkS") (width 0.12))
  (fp_line (start 3 1.72) (end 12.24 1.72) (layer "F.SilkS") (width 0.12))
  (fp_line (start 14.2 0) (end 12.24 0) (layer "F.SilkS") (width 0.12))
  (fp_line (start 1.04 0) (end 3 0) (layer "F.SilkS") (width 0.12))
  (pad "1" thru_hole circle (at 0 0 90) (size 1.6 1.6) (drill 0.8) (layers *.Cu *.Mask) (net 5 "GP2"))
  (pad "2" thru_hole oval (at 15.24 0 90) (size 1.6 1.6) (drill 0.8) (layers *.Cu *.Mask) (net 11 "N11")))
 (gr_arc (start 147 72) (mid 151.242641 73.757359) (end 153 78) (layer "Edge.Cuts") (width 0.1))
 (gr_line (start 147 72) (end 117 72) (layer "Edge.Cuts") (width 0.1))
 (gr_line (start 153 78) (end 153 108) (layer "Edge.Cuts") (width 0.1))
 (gr_line (start 111 78) (end 111 108) (layer "Edge.Cuts") (width 0.1))
 (gr_arc (start 111 78) (mid 112.757359 73.757359) (end 117 72) (layer "Edge.Cuts") (width 0.1))
 (gr_arc (start 153 108) (mid 151.242641 112.242641) (end 147 114) (layer "Edge.Cuts") (width 0.1))
 (gr_arc (start 117 114) (mid 112.757359 112.242641) (end 111 108) (layer "Edge.Cuts") (width 0.1))
 (gr_line (start 147 114) (end 117 114) (layer "Edge.Cuts") (width 0.1))
 (segment (start 117 108) (end 120.5 111.5) (width 0.5) (layer "F.Cu") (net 2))
 (segment (start 145.735 98) (end 145.735 106.735) (width 0.5) (layer "F.Cu") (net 2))
 (segment (start 122.52 93.16) (end 121.6 94.08) (width 0.5) (layer "F.Cu") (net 2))
 (segment (start 121.6 94.08) (end 117 89.48) (width 0.5) (layer "F.Cu") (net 2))
 (segment (start 145.835 97.9) (end 145.735 98) (width 0.5) (layer "F.Cu") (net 2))
 (segment (start 117 77.9) (end 120.5 74.4) (width 0.5) (layer "F.Cu") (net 2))
 (segment (start 145.835 79.065) (end 147 77.9) (width 0.5) (layer "F.Cu") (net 2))
 (segment (start 120.5 111.5) (end 143.5 111.5) (width 0.5) (layer "F.Cu") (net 2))
 (segment (start 143.5 111.5) (end 147 108) (width 0.5) (layer "F.Cu") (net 2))
 (segment (start 147.9 107.1) (end 147 108) (width 0.5) (layer "F.Cu") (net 2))
 (segment (start 138.25 104.25) (end 142 108) (width 0.5) (layer "F.Cu") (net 2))
 (segment (start 142 108) (end 147 108) (width 0.5) (layer "F.Cu") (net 2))
 (segment (start 129.74 86.26) (end 134.25 81.75) (width 0.5) (layer "F.Cu") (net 2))
 (segment (start 134.25 104.25) (end 138.25 104.25) (width 0.5) (layer "F.Cu") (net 2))
 (segment (start 120.5 74.4) (end 143.5 74.4) (width 0.5) (layer "F.Cu") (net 2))
 (segment (start 125.77 93.16) (end 122.52 93.16) (width 0.5) (layer "F.Cu") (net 2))
 (segment (start 143.5 74.4) (end 147 77.9) (width 0.5) (layer "F.Cu") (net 2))
 (segment (start 145.835 88.4) (end 145.835 97.9) (width 0.5) (layer "F.Cu") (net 2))
 (segment (start 117 89.48) (end 117 77.9) (width 0.5) (layer "F.Cu") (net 2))
 (segment (start 148 78.9) (end 147 77.9) (width 0.5) (layer "F.Cu") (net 2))
 (segment (start 129.74 89.18) (end 129.74 86.26) (width 0.5) (layer "F.Cu") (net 2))
 (segment (start 145.735 106.735) (end 147 108) (width 0.5) (layer "F.Cu") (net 2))
 (segment (start 145.835 88.4) (end 145.835 79.065) (width 0.5) (layer "F.Cu") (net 2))
 (via (at 125.77 93.16) (size 0.8) (drill 0.4) (layers "F.Cu" "B.Cu") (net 2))
 (segment (start 125.77 93.15) (end 125.77 93.16) (width 0.5) (layer "B.Cu") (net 2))
 (segment (start 129.74 89.18) (end 125.77 93.15) (width 0.5) (layer "B.Cu") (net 2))
 (segment (start 138.83 100.62) (end 138.83 97.17) (width 0.5) (layer "F.Cu") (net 9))
 (segment (start 143.295 92.705) (end 143.295 88.4) (width 0.5) (layer "F.Cu") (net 9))
 (segment (start 138.83 97.17) (end 143.295 92.705) (width 0.5) (layer "F.Cu") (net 9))
 (segment (start 143.195 95.805) (end 150.37 88.63) (width 0.5) (layer "B.Cu") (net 11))
 (segment (start 150.37 88.63) (end 150.37 85.33) (width 0.5) (layer "B.Cu") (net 11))
 (segment (start 143.195 98) (end 143.195 95.805) (width 0.5) (layer "B.Cu") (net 11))
 (segment (start 138.83 92.79) (end 134.82 96.8) (width 0.5) (layer "F.Cu") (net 6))
 (segment (start 138.83 85.38) (end 138.83 92.79) (width 0.5) (layer "F.Cu") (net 6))
 (segment (start 126.51 84.09) (end 137.54 84.09) (width 0.5) (layer "B.Cu") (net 6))
 (segment (start 137.54 84.09) (end 138.83 85.38) (width 0.5) (layer "B.Cu") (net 6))
 (segment (start 121.6 89) (end 126.51 84.09) (width 0.5) (layer "B.Cu") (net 6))
 (segment (start 134.82 89.18) (end 137 87) (width 0.5) (layer "F.Cu") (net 7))
 (segment (start 137 79.62) (end 139.62 77) (width 0.5) (layer "F.Cu") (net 7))
 (segment (start 132.46 91.54) (end 121.6 91.54) (width 0.5) (layer "F.Cu") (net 7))
 (segment (start 137 87) (end 137 79.62) (width 0.5) (layer "F.Cu") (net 7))
 (segment (start 134.82 89.18) (end 132.46 91.54) (width 0.5) (layer "F.Cu") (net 7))
 (segment (start 127.91 94.97) (end 123.25 94.97) (width 0.5) (layer "F.Cu") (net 4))
 (segment (start 123.25 94.97) (end 121.6 96.62) (width 0.5) (layer "F.Cu") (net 4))
 (segment (start 129.74 96.8) (end 127.91 94.97) (width 0.5) (layer "F.Cu") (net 4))
 (segment (start 124.38 101.94) (end 121.6 99.16) (width 0.5) (layer "F.Cu") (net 8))
 (segment (start 124.38 109) (end 124.38 101.94) (width 0.5) (layer "F.Cu") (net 8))
 (segment (start 124.46 91.92) (end 127.2 89.18) (width 0.5) (layer "B.Cu") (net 8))
 (segment (start 121.6 99.16) (end 124.46 96.3) (width 0.5) (layer "B.Cu") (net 8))
 (segment (start 124.46 96.3) (end 124.46 91.92) (width 0.5) (layer "B.Cu") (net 8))
 (segment (start 132.28 100.28) (end 135 103) (width 0.5) (layer "B.Cu") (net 5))
 (segment (start 147.94 103) (end 150.37 100.57) (width 0.5) (layer "B.Cu") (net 5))
 (segment (start 135 103) (end 147.94 103) (width 0.5) (layer "B.Cu") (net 5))
 (segment (start 132.28 96.8) (end 132.28 100.28) (width 0.5) (layer "B.Cu") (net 5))
 (segment (start 127.75 80.37) (end 124.38 77) (width 0.5) (layer "F.Cu") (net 1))
 (segment (start 127.75 81.75) (end 127.75 80.37) (width 0.5) (layer "F.Cu") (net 1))
 (segment (start 127.75 104.25) (end 132.5 109) (width 0.5) (layer "F.Cu") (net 3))
 (segment (start 132.5 109) (end 139.62 109) (width 0.5) (layer "F.Cu") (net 3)))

